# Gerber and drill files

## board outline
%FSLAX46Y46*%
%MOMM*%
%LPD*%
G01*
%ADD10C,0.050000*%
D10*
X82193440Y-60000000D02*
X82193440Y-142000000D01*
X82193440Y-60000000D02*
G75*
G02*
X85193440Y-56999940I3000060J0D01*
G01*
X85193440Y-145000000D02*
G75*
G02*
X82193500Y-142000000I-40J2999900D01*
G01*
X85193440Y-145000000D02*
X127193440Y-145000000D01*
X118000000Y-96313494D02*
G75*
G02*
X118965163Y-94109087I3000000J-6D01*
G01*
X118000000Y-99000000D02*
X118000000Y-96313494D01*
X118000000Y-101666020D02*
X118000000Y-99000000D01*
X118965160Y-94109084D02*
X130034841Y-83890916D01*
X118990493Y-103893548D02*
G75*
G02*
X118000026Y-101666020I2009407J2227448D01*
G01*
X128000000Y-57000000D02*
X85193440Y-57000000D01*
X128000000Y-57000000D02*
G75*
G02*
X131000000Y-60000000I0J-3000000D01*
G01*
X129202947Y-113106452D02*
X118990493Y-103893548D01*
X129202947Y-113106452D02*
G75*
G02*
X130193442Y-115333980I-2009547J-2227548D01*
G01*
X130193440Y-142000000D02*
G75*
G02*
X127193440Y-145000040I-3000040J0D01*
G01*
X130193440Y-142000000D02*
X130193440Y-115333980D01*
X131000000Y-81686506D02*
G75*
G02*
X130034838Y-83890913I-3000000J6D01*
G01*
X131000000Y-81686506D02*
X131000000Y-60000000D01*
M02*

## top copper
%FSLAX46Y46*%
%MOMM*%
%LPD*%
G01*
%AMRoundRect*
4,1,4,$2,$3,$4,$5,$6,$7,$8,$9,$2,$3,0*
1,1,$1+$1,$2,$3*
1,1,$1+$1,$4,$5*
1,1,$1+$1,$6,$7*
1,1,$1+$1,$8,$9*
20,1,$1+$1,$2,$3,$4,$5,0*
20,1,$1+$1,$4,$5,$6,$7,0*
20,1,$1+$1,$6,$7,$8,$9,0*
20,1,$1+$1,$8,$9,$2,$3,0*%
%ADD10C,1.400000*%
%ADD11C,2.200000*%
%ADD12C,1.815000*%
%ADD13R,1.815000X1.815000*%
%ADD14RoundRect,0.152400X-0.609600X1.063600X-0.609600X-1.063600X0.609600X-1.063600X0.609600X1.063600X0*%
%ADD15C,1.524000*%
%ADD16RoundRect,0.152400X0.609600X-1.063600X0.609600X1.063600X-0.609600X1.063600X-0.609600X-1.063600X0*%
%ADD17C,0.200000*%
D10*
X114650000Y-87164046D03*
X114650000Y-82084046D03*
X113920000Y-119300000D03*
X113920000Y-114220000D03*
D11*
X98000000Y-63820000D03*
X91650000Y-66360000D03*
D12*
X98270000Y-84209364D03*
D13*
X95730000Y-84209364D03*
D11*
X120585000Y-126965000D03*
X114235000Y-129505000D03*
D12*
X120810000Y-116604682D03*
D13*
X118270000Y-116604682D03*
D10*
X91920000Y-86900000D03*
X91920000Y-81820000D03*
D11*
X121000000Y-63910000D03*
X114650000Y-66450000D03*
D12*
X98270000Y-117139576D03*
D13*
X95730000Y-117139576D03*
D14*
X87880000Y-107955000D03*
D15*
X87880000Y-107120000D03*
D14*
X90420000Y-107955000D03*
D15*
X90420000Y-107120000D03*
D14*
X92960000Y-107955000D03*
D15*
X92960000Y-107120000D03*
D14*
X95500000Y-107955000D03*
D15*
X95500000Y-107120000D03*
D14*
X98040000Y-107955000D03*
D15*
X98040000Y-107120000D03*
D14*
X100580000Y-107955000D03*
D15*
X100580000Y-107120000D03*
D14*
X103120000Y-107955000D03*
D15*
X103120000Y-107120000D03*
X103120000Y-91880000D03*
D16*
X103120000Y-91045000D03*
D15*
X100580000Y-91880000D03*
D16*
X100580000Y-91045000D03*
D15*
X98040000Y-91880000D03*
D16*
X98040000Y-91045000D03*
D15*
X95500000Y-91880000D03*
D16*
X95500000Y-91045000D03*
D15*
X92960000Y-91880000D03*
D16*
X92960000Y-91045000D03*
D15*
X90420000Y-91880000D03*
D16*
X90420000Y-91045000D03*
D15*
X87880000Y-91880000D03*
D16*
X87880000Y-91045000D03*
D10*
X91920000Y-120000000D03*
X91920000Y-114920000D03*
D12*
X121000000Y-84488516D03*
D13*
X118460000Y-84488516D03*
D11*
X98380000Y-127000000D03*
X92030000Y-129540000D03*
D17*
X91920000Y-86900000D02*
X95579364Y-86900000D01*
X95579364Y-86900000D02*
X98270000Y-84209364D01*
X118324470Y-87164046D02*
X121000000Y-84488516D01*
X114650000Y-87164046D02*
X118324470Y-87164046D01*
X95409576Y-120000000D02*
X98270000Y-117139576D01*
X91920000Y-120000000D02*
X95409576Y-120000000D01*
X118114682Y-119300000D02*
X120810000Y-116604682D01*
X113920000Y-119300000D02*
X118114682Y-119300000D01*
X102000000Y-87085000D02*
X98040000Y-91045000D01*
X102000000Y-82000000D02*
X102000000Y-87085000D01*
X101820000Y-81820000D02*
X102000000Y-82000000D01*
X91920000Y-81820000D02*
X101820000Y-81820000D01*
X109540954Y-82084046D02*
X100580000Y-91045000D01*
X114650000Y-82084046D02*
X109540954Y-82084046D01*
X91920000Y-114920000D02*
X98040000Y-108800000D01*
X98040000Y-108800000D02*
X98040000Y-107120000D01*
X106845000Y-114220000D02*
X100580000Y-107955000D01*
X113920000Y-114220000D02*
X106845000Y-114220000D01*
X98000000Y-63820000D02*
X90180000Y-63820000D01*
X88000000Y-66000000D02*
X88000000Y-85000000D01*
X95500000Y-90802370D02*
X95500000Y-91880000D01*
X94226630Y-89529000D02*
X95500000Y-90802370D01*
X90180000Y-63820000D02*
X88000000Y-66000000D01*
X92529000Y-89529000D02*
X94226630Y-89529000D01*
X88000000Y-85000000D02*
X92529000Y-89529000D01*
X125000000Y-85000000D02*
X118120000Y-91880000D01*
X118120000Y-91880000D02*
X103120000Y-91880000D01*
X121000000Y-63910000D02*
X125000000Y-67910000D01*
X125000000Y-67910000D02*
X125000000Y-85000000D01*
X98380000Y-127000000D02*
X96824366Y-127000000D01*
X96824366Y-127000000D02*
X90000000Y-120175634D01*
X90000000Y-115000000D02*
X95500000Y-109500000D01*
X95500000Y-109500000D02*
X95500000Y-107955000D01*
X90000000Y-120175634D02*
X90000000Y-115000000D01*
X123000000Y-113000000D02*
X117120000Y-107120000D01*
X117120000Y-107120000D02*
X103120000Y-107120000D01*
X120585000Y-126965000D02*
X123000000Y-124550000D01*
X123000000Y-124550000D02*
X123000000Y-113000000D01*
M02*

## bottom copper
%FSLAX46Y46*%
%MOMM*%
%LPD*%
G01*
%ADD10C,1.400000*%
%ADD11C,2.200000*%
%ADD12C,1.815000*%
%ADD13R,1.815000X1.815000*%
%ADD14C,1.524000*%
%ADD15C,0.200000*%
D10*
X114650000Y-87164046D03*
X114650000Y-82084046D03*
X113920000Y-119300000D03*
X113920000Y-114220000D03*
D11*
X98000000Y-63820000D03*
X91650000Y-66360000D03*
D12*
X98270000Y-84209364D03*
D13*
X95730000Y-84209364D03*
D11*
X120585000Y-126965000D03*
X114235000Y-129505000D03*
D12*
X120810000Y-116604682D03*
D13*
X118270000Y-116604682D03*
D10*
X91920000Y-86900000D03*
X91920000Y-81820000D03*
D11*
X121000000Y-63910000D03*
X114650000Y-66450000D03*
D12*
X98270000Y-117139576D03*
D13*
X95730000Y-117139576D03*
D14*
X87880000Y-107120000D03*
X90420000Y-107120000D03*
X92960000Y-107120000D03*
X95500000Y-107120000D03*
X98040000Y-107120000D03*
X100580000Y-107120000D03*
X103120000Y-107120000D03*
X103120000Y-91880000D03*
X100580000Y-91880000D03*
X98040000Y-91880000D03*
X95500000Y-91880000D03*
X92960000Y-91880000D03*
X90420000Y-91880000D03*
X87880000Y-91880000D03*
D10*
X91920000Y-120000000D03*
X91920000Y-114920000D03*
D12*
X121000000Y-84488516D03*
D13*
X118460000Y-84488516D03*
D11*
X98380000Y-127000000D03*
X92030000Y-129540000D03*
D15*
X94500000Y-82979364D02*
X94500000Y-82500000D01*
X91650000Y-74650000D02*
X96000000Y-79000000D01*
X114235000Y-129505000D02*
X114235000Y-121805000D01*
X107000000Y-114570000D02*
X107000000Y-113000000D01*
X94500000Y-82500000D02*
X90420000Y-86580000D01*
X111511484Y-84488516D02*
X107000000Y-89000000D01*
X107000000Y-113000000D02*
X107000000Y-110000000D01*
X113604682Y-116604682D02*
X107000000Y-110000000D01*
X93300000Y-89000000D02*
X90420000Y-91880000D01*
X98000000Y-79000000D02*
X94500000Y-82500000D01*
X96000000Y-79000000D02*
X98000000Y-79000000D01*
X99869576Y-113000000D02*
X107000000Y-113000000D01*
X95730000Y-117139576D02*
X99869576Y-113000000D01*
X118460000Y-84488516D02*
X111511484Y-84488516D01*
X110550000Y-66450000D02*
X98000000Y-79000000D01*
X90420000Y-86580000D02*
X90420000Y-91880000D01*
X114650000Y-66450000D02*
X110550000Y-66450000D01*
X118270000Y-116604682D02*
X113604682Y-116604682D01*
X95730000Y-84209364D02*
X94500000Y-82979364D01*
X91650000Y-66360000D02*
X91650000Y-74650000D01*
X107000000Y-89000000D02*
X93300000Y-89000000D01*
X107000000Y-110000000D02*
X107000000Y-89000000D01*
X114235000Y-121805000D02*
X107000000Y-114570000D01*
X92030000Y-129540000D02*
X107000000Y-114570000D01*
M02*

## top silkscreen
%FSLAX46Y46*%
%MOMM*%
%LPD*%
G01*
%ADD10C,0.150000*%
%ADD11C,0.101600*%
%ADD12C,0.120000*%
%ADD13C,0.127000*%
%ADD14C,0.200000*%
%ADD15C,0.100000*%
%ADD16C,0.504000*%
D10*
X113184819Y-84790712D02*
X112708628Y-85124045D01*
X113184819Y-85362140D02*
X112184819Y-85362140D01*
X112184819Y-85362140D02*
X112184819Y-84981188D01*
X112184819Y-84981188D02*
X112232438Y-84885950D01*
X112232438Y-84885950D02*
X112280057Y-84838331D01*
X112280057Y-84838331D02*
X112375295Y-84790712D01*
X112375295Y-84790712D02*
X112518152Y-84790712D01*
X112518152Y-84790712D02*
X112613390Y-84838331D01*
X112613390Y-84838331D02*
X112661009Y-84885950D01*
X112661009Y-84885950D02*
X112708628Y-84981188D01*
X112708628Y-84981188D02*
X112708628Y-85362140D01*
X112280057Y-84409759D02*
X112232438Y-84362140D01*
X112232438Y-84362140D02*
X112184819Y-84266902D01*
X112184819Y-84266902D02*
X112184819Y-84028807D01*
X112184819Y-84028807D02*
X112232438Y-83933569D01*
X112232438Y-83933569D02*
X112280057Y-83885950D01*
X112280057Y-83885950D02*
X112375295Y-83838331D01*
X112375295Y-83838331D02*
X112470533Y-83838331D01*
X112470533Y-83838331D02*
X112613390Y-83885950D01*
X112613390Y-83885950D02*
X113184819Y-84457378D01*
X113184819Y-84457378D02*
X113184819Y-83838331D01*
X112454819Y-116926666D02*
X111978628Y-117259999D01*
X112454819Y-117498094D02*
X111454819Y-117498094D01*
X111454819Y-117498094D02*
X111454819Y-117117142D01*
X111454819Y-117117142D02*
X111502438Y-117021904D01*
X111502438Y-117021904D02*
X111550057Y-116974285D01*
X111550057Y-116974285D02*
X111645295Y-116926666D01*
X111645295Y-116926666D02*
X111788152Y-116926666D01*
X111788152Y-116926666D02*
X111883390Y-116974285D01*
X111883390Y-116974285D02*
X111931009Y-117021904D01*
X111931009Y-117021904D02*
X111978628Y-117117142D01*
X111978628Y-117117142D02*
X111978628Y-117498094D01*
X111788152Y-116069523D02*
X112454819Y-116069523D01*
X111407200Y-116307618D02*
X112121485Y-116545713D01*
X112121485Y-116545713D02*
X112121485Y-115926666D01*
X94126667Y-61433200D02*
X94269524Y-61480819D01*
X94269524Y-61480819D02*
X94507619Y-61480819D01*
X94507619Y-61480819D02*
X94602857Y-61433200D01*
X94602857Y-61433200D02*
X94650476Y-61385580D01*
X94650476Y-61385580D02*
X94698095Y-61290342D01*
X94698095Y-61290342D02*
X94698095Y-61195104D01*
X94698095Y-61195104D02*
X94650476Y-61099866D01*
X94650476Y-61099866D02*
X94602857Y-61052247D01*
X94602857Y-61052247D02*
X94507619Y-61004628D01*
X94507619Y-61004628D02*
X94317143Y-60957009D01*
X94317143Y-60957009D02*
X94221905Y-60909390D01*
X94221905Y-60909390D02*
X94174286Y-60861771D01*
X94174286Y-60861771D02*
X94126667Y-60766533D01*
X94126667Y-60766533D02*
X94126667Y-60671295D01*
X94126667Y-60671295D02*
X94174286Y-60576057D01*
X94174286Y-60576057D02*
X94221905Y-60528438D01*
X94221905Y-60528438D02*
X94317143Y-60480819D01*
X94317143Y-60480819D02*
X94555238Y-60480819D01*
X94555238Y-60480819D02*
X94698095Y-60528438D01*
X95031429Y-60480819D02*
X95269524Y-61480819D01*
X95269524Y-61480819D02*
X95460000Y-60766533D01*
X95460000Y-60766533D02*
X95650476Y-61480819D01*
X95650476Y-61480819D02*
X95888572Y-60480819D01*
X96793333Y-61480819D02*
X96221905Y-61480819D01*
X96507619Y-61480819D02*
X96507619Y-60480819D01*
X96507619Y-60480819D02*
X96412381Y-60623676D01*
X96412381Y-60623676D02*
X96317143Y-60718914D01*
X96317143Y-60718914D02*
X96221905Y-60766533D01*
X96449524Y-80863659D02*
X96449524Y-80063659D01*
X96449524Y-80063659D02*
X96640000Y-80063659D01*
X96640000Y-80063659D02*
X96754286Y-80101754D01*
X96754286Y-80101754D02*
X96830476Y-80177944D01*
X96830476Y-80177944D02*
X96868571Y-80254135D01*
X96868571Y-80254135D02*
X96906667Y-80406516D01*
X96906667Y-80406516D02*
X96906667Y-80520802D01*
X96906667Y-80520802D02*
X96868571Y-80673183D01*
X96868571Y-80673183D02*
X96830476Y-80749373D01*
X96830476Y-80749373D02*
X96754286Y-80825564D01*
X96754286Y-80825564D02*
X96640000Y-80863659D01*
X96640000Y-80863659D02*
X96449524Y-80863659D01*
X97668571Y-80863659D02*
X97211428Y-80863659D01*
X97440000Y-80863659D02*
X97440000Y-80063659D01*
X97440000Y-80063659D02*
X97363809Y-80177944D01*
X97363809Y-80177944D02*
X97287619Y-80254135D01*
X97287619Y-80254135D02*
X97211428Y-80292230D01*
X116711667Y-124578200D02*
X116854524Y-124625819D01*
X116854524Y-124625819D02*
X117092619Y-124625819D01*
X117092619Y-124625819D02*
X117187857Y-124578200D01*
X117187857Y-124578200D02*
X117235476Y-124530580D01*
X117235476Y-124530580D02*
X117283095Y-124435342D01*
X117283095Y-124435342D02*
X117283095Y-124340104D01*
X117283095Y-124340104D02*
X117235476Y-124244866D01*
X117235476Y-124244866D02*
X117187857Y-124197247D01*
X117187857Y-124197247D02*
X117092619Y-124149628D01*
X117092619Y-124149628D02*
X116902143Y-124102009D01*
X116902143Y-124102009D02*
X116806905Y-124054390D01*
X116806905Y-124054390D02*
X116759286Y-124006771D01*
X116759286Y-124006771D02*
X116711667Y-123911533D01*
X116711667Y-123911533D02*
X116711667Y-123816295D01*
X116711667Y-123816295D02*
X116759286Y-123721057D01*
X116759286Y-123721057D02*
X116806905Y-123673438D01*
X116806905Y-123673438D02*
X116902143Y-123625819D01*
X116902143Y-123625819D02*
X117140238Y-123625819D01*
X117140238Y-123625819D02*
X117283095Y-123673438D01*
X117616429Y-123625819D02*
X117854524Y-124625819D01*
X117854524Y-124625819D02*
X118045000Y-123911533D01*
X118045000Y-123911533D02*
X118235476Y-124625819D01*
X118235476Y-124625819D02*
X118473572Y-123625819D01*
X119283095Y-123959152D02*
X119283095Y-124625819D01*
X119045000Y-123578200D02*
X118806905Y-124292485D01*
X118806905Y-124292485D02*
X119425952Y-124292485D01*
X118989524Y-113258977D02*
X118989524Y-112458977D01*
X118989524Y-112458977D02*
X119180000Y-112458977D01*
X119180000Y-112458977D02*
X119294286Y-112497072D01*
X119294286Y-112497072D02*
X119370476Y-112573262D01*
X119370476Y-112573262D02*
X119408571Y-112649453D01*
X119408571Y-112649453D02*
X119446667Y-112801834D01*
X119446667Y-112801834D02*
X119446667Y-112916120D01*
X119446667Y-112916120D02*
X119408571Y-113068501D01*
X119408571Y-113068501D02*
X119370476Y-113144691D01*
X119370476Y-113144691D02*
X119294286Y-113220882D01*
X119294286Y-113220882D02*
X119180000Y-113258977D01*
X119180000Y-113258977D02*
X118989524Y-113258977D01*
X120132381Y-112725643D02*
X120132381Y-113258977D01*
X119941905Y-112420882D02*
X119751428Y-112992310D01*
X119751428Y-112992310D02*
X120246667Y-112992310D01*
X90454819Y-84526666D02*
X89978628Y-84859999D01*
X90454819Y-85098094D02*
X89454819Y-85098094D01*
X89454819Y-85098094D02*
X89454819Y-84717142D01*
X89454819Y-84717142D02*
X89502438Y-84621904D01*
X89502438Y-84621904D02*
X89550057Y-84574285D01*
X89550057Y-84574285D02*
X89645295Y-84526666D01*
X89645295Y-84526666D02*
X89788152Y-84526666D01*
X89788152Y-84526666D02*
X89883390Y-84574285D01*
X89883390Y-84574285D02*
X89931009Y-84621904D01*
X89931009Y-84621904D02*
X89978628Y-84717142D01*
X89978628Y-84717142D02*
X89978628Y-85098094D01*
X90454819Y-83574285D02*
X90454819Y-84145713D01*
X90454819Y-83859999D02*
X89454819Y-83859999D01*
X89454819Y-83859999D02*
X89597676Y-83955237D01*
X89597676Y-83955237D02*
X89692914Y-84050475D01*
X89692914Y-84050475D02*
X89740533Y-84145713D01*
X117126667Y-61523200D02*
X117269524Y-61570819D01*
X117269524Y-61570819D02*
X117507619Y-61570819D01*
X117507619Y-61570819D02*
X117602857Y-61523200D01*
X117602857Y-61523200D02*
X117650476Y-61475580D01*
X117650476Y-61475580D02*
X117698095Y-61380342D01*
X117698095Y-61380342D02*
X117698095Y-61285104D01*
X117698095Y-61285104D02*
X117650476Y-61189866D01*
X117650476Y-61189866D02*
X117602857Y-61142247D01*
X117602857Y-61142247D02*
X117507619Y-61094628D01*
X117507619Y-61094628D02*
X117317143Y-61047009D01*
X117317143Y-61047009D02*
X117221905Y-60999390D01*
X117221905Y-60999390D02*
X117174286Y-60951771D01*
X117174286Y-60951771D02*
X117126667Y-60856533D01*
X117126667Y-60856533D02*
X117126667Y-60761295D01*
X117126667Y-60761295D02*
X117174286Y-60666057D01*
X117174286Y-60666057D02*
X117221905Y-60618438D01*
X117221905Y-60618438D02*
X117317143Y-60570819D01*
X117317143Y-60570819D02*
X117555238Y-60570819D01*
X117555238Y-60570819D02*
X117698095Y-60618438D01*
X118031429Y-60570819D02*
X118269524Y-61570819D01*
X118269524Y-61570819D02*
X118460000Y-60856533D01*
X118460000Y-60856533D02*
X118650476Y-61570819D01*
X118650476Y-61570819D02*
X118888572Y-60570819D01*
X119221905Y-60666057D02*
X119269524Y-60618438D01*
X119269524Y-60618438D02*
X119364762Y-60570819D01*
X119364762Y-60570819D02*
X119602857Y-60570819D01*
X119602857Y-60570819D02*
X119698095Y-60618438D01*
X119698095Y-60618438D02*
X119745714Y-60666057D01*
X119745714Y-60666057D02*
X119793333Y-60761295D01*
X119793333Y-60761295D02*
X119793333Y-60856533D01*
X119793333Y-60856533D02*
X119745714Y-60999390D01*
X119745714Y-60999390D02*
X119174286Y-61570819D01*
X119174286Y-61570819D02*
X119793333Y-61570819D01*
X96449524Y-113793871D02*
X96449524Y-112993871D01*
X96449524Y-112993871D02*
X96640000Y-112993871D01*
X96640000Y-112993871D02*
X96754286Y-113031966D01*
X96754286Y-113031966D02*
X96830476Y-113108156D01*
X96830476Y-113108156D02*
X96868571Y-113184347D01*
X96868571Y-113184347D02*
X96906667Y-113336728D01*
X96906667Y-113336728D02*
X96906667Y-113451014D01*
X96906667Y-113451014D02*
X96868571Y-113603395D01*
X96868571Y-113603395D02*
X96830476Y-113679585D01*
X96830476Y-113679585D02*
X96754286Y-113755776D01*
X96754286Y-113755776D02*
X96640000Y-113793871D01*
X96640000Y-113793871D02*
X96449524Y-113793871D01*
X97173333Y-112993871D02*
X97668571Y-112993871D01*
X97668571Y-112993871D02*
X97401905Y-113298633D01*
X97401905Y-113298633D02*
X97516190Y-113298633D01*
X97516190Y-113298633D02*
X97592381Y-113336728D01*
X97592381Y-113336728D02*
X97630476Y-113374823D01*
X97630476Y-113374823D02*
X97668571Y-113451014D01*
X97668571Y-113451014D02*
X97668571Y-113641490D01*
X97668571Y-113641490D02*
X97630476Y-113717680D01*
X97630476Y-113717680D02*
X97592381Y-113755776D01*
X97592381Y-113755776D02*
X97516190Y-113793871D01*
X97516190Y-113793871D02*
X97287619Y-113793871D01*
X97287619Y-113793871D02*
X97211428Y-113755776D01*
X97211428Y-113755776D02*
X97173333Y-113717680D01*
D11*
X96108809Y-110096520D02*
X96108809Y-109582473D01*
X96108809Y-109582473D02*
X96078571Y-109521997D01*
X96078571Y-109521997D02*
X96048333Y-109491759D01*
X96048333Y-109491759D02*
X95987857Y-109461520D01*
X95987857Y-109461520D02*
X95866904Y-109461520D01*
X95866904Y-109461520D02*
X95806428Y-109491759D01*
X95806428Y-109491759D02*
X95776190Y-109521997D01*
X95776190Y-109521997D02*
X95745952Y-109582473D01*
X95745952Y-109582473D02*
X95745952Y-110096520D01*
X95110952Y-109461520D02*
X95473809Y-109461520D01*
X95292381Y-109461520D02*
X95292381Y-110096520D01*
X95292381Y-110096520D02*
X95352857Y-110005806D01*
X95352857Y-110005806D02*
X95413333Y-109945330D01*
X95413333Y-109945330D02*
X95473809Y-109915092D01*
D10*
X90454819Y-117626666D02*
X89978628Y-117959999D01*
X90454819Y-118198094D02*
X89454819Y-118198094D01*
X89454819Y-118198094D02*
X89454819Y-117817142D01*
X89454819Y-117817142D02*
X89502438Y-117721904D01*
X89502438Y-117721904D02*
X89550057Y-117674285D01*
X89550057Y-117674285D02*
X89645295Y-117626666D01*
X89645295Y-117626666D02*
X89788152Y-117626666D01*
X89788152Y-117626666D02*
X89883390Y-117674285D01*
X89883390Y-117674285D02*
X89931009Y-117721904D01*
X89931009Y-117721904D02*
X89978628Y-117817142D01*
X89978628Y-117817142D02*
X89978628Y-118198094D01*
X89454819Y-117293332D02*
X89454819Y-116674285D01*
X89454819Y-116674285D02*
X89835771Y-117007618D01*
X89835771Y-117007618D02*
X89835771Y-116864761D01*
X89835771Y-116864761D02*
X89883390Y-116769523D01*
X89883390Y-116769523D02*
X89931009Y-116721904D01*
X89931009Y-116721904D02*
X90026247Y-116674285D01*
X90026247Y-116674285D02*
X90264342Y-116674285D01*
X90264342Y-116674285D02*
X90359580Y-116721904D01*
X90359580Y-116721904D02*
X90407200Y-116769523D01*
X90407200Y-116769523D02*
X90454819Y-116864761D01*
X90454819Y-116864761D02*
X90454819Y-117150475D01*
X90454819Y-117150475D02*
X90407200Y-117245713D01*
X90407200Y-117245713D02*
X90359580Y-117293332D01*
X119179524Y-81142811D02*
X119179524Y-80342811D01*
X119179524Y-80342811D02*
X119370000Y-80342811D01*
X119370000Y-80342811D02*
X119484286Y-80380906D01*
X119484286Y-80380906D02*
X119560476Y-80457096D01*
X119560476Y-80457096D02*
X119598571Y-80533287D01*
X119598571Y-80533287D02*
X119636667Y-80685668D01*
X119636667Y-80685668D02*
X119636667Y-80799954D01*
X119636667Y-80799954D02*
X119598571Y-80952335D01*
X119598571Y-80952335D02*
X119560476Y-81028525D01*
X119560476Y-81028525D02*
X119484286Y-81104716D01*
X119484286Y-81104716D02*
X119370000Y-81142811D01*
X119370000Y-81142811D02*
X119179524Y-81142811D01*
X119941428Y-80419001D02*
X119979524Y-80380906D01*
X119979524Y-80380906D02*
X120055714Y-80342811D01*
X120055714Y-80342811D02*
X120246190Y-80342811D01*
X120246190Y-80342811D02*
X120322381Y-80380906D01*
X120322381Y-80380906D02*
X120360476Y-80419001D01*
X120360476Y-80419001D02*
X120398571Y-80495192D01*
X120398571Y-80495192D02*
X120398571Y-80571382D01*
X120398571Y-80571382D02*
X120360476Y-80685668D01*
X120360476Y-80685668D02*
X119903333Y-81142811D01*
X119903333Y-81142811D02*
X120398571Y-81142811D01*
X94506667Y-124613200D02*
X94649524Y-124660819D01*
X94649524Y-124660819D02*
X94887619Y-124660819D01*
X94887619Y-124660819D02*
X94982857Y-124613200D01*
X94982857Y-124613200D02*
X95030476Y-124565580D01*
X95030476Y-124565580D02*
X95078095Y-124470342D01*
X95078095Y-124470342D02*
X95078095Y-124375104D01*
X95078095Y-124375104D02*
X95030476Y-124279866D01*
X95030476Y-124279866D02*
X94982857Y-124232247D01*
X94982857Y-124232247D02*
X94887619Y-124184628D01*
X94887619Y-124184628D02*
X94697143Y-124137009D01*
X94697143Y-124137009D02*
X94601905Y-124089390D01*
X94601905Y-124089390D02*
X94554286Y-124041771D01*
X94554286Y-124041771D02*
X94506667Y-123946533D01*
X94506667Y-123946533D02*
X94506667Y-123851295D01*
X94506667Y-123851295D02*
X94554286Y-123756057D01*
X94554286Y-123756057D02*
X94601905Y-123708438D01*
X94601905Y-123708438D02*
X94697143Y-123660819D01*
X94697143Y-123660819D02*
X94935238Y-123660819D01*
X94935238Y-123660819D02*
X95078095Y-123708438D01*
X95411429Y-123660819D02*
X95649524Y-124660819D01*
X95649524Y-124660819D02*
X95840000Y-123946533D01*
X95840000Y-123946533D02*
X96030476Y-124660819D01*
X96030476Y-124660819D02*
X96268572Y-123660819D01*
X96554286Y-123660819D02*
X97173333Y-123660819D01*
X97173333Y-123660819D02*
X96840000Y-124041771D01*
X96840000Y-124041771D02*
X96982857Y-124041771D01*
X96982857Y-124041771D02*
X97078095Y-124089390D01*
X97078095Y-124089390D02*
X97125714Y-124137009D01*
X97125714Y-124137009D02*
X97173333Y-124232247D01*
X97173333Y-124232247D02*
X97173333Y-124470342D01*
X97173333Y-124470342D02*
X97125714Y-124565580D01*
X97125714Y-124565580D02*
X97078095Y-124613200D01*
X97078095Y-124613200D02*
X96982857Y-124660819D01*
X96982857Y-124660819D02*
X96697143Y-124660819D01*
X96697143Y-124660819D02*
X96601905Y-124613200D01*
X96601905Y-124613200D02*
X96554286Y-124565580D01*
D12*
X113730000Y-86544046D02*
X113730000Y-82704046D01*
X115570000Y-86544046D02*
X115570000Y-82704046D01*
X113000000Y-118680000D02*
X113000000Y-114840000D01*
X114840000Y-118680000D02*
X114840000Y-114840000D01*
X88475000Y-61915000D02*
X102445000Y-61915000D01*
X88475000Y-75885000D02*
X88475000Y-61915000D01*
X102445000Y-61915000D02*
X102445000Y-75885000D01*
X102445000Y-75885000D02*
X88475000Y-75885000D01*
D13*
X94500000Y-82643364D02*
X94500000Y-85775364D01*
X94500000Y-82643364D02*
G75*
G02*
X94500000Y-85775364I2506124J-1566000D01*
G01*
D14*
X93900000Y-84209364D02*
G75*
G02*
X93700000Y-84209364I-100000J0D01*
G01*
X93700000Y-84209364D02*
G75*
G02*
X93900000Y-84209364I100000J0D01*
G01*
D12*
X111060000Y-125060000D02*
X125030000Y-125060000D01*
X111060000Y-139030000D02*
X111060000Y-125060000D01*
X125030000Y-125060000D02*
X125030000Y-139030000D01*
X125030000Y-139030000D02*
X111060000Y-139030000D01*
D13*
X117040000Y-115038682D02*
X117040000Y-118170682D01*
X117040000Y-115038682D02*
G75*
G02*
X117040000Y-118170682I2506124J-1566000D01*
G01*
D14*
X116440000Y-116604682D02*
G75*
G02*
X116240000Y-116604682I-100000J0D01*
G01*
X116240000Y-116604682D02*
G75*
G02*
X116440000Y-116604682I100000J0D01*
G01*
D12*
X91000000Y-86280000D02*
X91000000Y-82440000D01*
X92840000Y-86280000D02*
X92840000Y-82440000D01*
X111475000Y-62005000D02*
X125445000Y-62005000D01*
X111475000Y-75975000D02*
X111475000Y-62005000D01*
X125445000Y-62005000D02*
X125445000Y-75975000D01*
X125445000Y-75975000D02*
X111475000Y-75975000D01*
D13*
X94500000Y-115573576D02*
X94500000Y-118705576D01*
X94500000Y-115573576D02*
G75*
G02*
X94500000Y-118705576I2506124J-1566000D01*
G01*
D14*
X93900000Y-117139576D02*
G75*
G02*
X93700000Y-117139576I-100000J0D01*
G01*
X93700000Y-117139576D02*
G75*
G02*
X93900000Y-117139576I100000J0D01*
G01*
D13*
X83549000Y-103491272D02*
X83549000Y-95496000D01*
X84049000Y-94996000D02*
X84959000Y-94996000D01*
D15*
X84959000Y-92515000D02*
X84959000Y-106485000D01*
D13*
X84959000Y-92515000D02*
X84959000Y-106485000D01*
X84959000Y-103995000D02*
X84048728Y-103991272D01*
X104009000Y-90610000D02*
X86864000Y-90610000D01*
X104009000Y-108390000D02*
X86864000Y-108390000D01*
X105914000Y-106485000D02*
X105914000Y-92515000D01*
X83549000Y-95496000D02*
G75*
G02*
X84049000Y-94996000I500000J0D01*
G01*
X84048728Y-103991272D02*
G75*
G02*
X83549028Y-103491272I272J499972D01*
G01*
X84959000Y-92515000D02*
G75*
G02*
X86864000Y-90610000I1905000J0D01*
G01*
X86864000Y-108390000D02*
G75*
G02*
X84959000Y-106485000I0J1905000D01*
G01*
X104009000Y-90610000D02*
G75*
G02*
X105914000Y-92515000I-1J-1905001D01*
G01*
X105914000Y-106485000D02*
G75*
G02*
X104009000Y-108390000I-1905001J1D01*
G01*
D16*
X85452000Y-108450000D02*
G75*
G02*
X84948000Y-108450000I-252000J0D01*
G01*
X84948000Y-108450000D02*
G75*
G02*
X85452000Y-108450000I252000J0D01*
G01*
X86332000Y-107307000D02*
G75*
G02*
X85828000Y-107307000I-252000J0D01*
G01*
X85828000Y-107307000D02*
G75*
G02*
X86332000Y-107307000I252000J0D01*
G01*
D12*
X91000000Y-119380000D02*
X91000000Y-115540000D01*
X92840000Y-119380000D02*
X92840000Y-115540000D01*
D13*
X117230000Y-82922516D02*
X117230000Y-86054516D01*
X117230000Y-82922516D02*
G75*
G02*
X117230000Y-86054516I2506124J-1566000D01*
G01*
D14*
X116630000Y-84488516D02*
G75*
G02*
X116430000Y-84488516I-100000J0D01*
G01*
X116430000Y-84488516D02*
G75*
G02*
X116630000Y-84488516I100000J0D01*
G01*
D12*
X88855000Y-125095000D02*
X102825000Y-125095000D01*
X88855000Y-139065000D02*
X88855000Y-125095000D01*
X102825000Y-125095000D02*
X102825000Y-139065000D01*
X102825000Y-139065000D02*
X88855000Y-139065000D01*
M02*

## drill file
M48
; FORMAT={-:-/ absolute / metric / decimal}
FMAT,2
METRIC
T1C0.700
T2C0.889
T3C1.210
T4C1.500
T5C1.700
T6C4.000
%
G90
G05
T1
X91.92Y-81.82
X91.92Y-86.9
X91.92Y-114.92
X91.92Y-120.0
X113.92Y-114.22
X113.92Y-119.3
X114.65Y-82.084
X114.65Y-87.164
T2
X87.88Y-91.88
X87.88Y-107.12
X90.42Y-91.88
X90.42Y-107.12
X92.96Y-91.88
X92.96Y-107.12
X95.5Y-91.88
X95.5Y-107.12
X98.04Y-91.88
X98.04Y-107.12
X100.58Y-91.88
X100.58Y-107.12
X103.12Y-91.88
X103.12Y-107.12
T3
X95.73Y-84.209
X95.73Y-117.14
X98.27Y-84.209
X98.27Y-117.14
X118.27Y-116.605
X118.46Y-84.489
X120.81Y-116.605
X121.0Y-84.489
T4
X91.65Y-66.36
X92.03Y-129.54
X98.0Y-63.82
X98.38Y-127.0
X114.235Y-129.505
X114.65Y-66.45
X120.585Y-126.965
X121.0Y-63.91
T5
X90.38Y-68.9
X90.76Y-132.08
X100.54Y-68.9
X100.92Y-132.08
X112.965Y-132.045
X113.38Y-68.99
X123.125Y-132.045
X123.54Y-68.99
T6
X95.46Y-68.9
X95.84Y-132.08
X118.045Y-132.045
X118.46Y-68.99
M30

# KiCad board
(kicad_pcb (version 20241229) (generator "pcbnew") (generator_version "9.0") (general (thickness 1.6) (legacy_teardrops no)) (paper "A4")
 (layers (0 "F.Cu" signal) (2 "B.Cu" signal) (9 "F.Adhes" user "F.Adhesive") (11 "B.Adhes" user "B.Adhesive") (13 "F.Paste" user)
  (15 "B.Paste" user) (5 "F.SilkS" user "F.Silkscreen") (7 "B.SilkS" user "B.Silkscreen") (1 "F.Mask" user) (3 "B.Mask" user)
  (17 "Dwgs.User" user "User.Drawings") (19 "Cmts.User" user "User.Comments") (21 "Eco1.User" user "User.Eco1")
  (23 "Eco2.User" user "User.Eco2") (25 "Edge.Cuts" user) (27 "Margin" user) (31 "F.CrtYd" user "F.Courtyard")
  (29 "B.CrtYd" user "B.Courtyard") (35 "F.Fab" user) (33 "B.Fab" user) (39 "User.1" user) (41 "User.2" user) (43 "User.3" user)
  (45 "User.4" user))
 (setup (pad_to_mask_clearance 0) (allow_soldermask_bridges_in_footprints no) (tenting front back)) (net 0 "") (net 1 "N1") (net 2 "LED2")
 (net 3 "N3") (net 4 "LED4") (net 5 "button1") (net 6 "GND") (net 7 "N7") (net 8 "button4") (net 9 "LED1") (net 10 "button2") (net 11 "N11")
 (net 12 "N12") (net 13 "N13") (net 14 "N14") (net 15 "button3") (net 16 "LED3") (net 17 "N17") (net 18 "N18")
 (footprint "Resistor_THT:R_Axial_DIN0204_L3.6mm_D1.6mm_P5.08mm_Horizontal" (layer "F.Cu") (at 114.65 87.164046 90)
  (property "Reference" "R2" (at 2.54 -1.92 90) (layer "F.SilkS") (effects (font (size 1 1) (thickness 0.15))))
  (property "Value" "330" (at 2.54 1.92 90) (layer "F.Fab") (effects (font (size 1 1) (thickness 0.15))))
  (fp_line (start 0.62 -0.92) (end 4.46 -0.92) (stroke (width 0.12) (type solid)) (layer "F.SilkS"))
  (fp_line (start 0.62 0.92) (end 4.46 0.92) (stroke (width 0.12) (type solid)) (layer "F.SilkS"))
  (pad "1" thru_hole circle (at 0 0 90) (size 1.4 1.4) (drill 0.7) (layers "*.Cu" "*.Mask") (remove_unused_layers no) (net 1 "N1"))
  (pad "2" thru_hole circle (at 5.08 0 90) (size 1.4 1.4) (drill 0.7) (layers "*.Cu" "*.Mask") (remove_unused_layers no) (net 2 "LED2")))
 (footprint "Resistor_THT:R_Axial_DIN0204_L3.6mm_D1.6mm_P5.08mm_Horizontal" (layer "F.Cu") (at 113.92 119.3 90)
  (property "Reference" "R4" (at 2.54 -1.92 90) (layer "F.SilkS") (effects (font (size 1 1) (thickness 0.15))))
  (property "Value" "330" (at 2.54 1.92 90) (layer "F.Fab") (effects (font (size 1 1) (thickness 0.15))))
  (fp_line (start 0.62 -0.92) (end 4.46 -0.92) (stroke (width 0.12) (type solid)) (layer "F.SilkS"))
  (fp_line (start 0.62 0.92) (end 4.46 0.92) (stroke (width 0.12) (type solid)) (layer "F.SilkS"))
  (pad "1" thru_hole circle (at 0 0 90) (size 1.4 1.4) (drill 0.7) (layers "*.Cu" "*.Mask") (remove_unused_layers no) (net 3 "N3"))
  (pad "2" thru_hole circle (at 5.08 0 90) (size 1.4 1.4) (drill 0.7) (layers "*.Cu" "*.Mask") (remove_unused_layers no) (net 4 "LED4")))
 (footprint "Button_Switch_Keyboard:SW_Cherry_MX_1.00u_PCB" (layer "F.Cu") (at 98 63.82)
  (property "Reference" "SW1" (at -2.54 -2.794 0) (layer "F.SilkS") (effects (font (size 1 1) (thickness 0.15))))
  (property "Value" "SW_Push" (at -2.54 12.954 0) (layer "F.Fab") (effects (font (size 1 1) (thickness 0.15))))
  (fp_line (start -9.525 -1.905) (end 4.445 -1.905) (stroke (width 0.12) (type solid)) (layer "F.SilkS"))
  (fp_line (start -9.525 12.065) (end -9.525 -1.905) (stroke (width 0.12) (type solid)) (layer "F.SilkS"))
  (fp_line (start 4.445 -1.905) (end 4.445 12.065) (stroke (width 0.12) (type solid)) (layer "F.SilkS"))
  (fp_line (start 4.445 12.065) (end -9.525 12.065) (stroke (width 0.12) (type solid)) (layer "F.SilkS"))
  (pad "" np_thru_hole circle (at -7.62 5.08) (size 1.7 1.7) (drill 1.7) (layers "*.Cu" "*.Mask"))
  (pad "" np_thru_hole circle (at -2.54 5.08) (size 4 4) (drill 4) (layers "*.Cu" "*.Mask"))
  (pad "" np_thru_hole circle (at 2.54 5.08) (size 1.7 1.7) (drill 1.7) (layers "*.Cu" "*.Mask"))
  (pad "1" thru_hole circle (at 0 0) (size 2.2 2.2) (drill 1.5) (layers "*.Cu" "*.Mask") (remove_unused_layers no) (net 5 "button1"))
  (pad "2" thru_hole circle (at -6.35 2.54) (size 2.2 2.2) (drill 1.5) (layers "*.Cu" "*.Mask") (remove_unused_layers no) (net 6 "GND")))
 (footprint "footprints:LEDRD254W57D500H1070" (layer "F.Cu") (at 97 84.209364)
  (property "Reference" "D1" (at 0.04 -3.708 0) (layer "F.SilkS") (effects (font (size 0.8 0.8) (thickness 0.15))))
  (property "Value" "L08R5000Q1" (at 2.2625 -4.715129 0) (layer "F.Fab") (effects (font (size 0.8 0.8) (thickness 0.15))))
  (fp_line (start -2.5 -1.566) (end -2.5 1.566) (stroke (width 0.127) (type solid)) (layer "F.SilkS"))
  (fp_arc (start -2.5 -1.566) (mid 2.961291 0) (end -2.5 1.566) (stroke (width 0.127) (type solid)) (layer "F.SilkS"))
  (fp_circle (center -3.2 0) (end -3.1 0) (stroke (width 0.2) (type solid)) (fill no) (layer "F.SilkS"))
  (pad "A" thru_hole circle (at 1.27 0) (size 1.815 1.815) (drill 1.21) (layers "*.Cu" "*.Mask") (remove_unused_layers no) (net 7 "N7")
   (solder_mask_margin 0.102))
  (pad "C" thru_hole rect (at -1.27 0) (size 1.815 1.815) (drill 1.21) (layers "*.Cu" "*.Mask") (remove_unused_layers no) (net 6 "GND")
   (solder_mask_margin 0.102)))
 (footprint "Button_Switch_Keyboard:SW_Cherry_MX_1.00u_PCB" (layer "F.Cu") (at 120.585 126.965)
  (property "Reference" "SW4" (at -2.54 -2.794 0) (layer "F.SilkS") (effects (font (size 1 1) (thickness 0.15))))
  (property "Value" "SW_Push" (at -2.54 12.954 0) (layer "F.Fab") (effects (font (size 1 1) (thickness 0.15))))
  (fp_line (start -9.525 -1.905) (end 4.445 -1.905) (stroke (width 0.12) (type solid)) (layer "F.SilkS"))
  (fp_line (start -9.525 12.065) (end -9.525 -1.905) (stroke (width 0.12) (type solid)) (layer "F.SilkS"))
  (fp_line (start 4.445 -1.905) (end 4.445 12.065) (stroke (width 0.12) (type solid)) (layer "F.SilkS"))
  (fp_line (start 4.445 12.065) (end -9.525 12.065) (stroke (width 0.12) (type solid)) (layer "F.SilkS"))
  (pad "" np_thru_hole circle (at -7.62 5.08) (size 1.7 1.7) (drill 1.7) (layers "*.Cu" "*.Mask"))
  (pad "" np_thru_hole circle (at -2.54 5.08) (size 4 4) (drill 4) (layers "*.Cu" "*.Mask"))
  (pad "" np_thru_hole circle (at 2.54 5.08) (size 1.7 1.7) (drill 1.7) (layers "*.Cu" "*.Mask"))
  (pad "1" thru_hole circle (at 0 0) (size 2.2 2.2) (drill 1.5) (layers "*.Cu" "*.Mask") (remove_unused_layers no) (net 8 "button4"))
  (pad "2" thru_hole circle (at -6.35 2.54) (size 2.2 2.2) (drill 1.5) (layers "*.Cu" "*.Mask") (remove_unused_layers no) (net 6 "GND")))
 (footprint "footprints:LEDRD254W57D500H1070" (layer "F.Cu") (at 119.54 116.604682)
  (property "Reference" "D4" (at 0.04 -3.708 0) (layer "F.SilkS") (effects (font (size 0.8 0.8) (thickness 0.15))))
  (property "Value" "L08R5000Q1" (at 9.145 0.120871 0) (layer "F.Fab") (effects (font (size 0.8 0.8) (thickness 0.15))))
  (fp_line (start -2.5 -1.566) (end -2.5 1.566) (stroke (width 0.127) (type solid)) (layer "F.SilkS"))
  (fp_arc (start -2.5 -1.566) (mid 2.961291 0) (end -2.5 1.566) (stroke (width 0.127) (type solid)) (layer "F.SilkS"))
  (fp_circle (center -3.2 0) (end -3.1 0) (stroke (width 0.2) (type solid)) (fill no) (layer "F.SilkS"))
  (pad "A" thru_hole circle (at 1.27 0) (size 1.815 1.815) (drill 1.21) (layers "*.Cu" "*.Mask") (remove_unused_layers no) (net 3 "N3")
   (solder_mask_margin 0.102))
  (pad "C" thru_hole rect (at -1.27 0) (size 1.815 1.815) (drill 1.21) (layers "*.Cu" "*.Mask") (remove_unused_layers no) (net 6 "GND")
   (solder_mask_margin 0.102)))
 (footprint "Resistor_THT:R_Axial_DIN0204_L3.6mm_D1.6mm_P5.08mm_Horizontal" (layer "F.Cu") (at 91.92 86.9 90)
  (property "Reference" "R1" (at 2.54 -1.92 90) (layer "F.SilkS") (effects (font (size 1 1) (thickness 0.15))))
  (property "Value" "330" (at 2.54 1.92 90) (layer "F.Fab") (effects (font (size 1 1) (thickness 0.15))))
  (fp_line (start 0.62 -0.92) (end 4.46 -0.92) (stroke (width 0.12) (type solid)) (layer "F.SilkS"))
  (fp_line (start 0.62 0.92) (end 4.46 0.92) (stroke (width 0.12) (type solid)) (layer "F.SilkS"))
  (pad "1" thru_hole circle (at 0 0 90) (size 1.4 1.4) (drill 0.7) (layers "*.Cu" "*.Mask") (remove_unused_layers no) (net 7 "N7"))
  (pad "2" thru_hole circle (at 5.08 0 90) (size 1.4 1.4) (drill 0.7) (layers "*.Cu" "*.Mask") (remove_unused_layers no) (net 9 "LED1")))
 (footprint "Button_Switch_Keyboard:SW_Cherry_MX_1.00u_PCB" (layer "F.Cu") (at 121 63.91)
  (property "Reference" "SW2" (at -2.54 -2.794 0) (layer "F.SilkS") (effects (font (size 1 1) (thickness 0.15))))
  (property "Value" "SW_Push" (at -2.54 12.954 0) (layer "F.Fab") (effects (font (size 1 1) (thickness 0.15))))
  (fp_line (start -9.525 -1.905) (end 4.445 -1.905) (stroke (width 0.12) (type solid)) (layer "F.SilkS"))
  (fp_line (start -9.525 12.065) (end -9.525 -1.905) (stroke (width 0.12) (type solid)) (layer "F.SilkS"))
  (fp_line (start 4.445 -1.905) (end 4.445 12.065) (stroke (width 0.12) (type solid)) (layer "F.SilkS"))
  (fp_line (start 4.445 12.065) (end -9.525 12.065) (stroke (width 0.12) (type solid)) (layer "F.SilkS"))
  (pad "" np_thru_hole circle (at -7.62 5.08) (size 1.7 1.7) (drill 1.7) (layers "*.Cu" "*.Mask"))
  (pad "" np_thru_hole circle (at -2.54 5.08) (size 4 4) (drill 4) (layers "*.Cu" "*.Mask"))
  (pad "" np_thru_hole circle (at 2.54 5.08) (size 1.7 1.7) (drill 1.7) (layers "*.Cu" "*.Mask"))
  (pad "1" thru_hole circle (at 0 0) (size 2.2 2.2) (drill 1.5) (layers "*.Cu" "*.Mask") (remove_unused_layers no) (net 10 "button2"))
  (pad "2" thru_hole circle (at -6.35 2.54) (size 2.2 2.2) (drill 1.5) (layers "*.Cu" "*.Mask") (remove_unused_layers no) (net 6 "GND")))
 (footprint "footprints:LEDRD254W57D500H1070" (layer "F.Cu") (at 97 117.139576)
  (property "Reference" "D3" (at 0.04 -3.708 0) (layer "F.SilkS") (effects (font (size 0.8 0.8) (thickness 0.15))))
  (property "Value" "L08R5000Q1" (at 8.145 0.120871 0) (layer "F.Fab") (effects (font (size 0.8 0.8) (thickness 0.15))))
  (fp_line (start -2.5 -1.566) (end -2.5 1.566) (stroke (width 0.127) (type solid)) (layer "F.SilkS"))
  (fp_arc (start -2.5 -1.566) (mid 2.961291 0) (end -2.5 1.566) (stroke (width 0.127) (type solid)) (layer "F.SilkS"))
  (fp_circle (center -3.2 0) (end -3.1 0) (stroke (width 0.2) (type solid)) (fill no) (layer "F.SilkS"))
  (pad "A" thru_hole circle (at 1.27 0) (size 1.815 1.815) (drill 1.21) (layers "*.Cu" "*.Mask") (remove_unused_layers no) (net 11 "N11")
   (solder_mask_margin 0.102))
  (pad "C" thru_hole rect (at -1.27 0) (size 1.815 1.815) (drill 1.21) (layers "*.Cu" "*.Mask") (remove_unused_layers no) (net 6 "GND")
   (solder_mask_margin 0.102)))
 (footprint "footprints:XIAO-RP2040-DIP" (layer "F.Cu") (at 95.5 99.5 180)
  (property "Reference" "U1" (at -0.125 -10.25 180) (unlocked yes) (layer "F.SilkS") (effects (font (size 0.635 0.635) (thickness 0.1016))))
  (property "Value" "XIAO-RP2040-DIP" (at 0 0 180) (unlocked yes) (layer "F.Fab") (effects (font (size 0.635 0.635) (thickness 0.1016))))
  (fp_line (start 11.951 -3.991272) (end 11.951 4.004) (stroke (width 0.127) (type solid)) (layer "F.SilkS"))
  (fp_line (start 11.451 4.504) (end 10.541 4.504) (stroke (width 0.127) (type solid)) (layer "F.SilkS"))
  (fp_line (start 10.541 6.985) (end 10.541 -6.985) (stroke (width 0.1) (type solid)) (layer "F.SilkS"))
  (fp_line (start 10.541 6.985) (end 10.541 -6.985) (stroke (width 0.127) (type solid)) (layer "F.SilkS"))
  (fp_line (start 10.541 -4.495) (end 11.451272 -4.491272) (stroke (width 0.127) (type solid)) (layer "F.SilkS"))
  (fp_line (start -8.509 8.89) (end 8.636 8.89) (stroke (width 0.127) (type solid)) (layer "F.SilkS"))
  (fp_line (start -8.509 -8.89) (end 8.636 -8.89) (stroke (width 0.127) (type solid)) (layer "F.SilkS"))
  (fp_line (start -10.414 -6.985) (end -10.414 6.985) (stroke (width 0.127) (type solid)) (layer "F.SilkS"))
  (fp_arc (start 11.951 4.004) (mid 11.804553 4.357553) (end 11.451 4.504) (stroke (width 0.127) (type default)) (layer "F.SilkS"))
  (fp_arc (start 11.451272 -4.491272) (mid 11.804644 -4.344724) (end 11.951 -3.991272) (stroke (width 0.127) (type default))
   (layer "F.SilkS"))
  (fp_arc (start 10.541 6.985) (mid 9.983038 8.332038) (end 8.636 8.89) (stroke (width 0.127) (type solid)) (layer "F.SilkS"))
  (fp_arc (start 8.636 -8.89) (mid 9.983038 -8.332038) (end 10.541 -6.985) (stroke (width 0.127) (type solid)) (layer "F.SilkS"))
  (fp_arc (start -8.509 8.89) (mid -9.856038 8.332038) (end -10.414 6.985) (stroke (width 0.127) (type solid)) (layer "F.SilkS"))
  (fp_arc (start -10.414 -6.985) (mid -9.856038 -8.332038) (end -8.509 -8.89) (stroke (width 0.127) (type solid)) (layer "F.SilkS"))
  (fp_circle (center 10.3 -8.95) (end 10.554 -8.95) (stroke (width 0.5) (type solid)) (fill yes) (layer "F.SilkS"))
  (fp_circle (center 9.42 -7.807) (end 9.674 -7.807) (stroke (width 0.5) (type solid)) (fill yes) (layer "F.SilkS"))
  (pad "1" smd roundrect (at 7.62 -8.455 270) (size 2.432 1.524) (layers "F.Cu" "F.Mask") (roundrect_rratio 0.1) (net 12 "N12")
   (thermal_bridge_angle 45))
  (pad "1" thru_hole circle (at 7.62 -7.62 270) (size 1.524 1.524) (drill 0.889) (layers "*.Cu" "*.Mask") (remove_unused_layers no)
   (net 12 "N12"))
  (pad "2" smd roundrect (at 5.08 -8.455 270) (size 2.432 1.524) (layers "F.Cu" "F.Mask") (roundrect_rratio 0.1) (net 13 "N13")
   (thermal_bridge_angle 45))
  (pad "2" thru_hole circle (at 5.08 -7.62 270) (size 1.524 1.524) (drill 0.889) (layers "*.Cu" "*.Mask") (remove_unused_layers no)
   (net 13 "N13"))
  (pad "3" smd roundrect (at 2.54 -8.455 270) (size 2.432 1.524) (layers "F.Cu" "F.Mask") (roundrect_rratio 0.1) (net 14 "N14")
   (thermal_bridge_angle 45))
  (pad "3" thru_hole circle (at 2.54 -7.62 270) (size 1.524 1.524) (drill 0.889) (layers "*.Cu" "*.Mask") (remove_unused_layers no)
   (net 14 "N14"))
  (pad "4" smd roundrect (at 0 -8.455 270) (size 2.432 1.524) (layers "F.Cu" "F.Mask") (roundrect_rratio 0.1) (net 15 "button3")
   (thermal_bridge_angle 45))
  (pad "4" thru_hole circle (at 0 -7.62 270) (size 1.524 1.524) (drill 0.889) (layers "*.Cu" "*.Mask") (remove_unused_layers no)
   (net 15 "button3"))
  (pad "5" smd roundrect (at -2.54 -8.455 270) (size 2.432 1.524) (layers "F.Cu" "F.Mask") (roundrect_rratio 0.1) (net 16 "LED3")
   (thermal_bridge_angle 45))
  (pad "5" thru_hole circle (at -2.54 -7.62 270) (size 1.524 1.524) (drill 0.889) (layers "*.Cu" "*.Mask") (remove_unused_layers no)
   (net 16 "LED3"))
  (pad "6" smd roundrect (at -5.08 -8.455 270) (size 2.432 1.524) (layers "F.Cu" "F.Mask") (roundrect_rratio 0.1) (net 4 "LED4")
   (thermal_bridge_angle 45))
  (pad "6" thru_hole circle (at -5.08 -7.62 270) (size 1.524 1.524) (drill 0.889) (layers "*.Cu" "*.Mask") (remove_unused_layers no)
   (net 4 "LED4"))
  (pad "7" smd roundrect (at -7.62 -8.455 270) (size 2.432 1.524) (layers "F.Cu" "F.Mask") (roundrect_rratio 0.1) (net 8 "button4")
   (thermal_bridge_angle 45))
  (pad "7" thru_hole circle (at -7.62 -7.62 270) (size 1.524 1.524) (drill 0.889) (layers "*.Cu" "*.Mask") (remove_unused_layers no)
   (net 8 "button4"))
  (pad "8" thru_hole circle (at -7.62 7.62 90) (size 1.524 1.524) (drill 0.889) (layers "*.Cu" "*.Mask") (remove_unused_layers no)
   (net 10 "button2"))
  (pad "8" smd roundrect (at -7.62 8.455 90) (size 2.432 1.524) (layers "F.Cu" "F.Mask") (roundrect_rratio 0.1) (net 10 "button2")
   (thermal_bridge_angle 45))
  (pad "9" thru_hole circle (at -5.08 7.62 90) (size 1.524 1.524) (drill 0.889) (layers "*.Cu" "*.Mask") (remove_unused_layers no)
   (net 2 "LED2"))
  (pad "9" smd roundrect (at -5.08 8.455 90) (size 2.432 1.524) (layers "F.Cu" "F.Mask") (roundrect_rratio 0.1) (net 2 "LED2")
   (thermal_bridge_angle 45))
  (pad "10" thru_hole circle (at -2.54 7.62 90) (size 1.524 1.524) (drill 0.889) (layers "*.Cu" "*.Mask") (remove_unused_layers no)
   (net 9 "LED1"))
  (pad "10" smd roundrect (at -2.54 8.455 90) (size 2.432 1.524) (layers "F.Cu" "F.Mask") (roundrect_rratio 0.1) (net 9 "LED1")
   (thermal_bridge_angle 45))
  (pad "11" thru_hole circle (at 0 7.62 90) (size 1.524 1.524) (drill 0.889) (layers "*.Cu" "*.Mask") (remove_unused_layers no)
   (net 5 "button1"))
  (pad "11" smd roundrect (at 0 8.455 90) (size 2.432 1.524) (layers "F.Cu" "F.Mask") (roundrect_rratio 0.1) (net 5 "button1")
   (thermal_bridge_angle 45))
  (pad "12" thru_hole circle (at 2.54 7.62 90) (size 1.524 1.524) (drill 0.889) (layers "*.Cu" "*.Mask") (remove_unused_layers no)
   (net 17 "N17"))
  (pad "12" smd roundrect (at 2.54 8.455 90) (size 2.432 1.524) (layers "F.Cu" "F.Mask") (roundrect_rratio 0.1) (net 17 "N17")
   (thermal_bridge_angle 45))
  (pad "13" thru_hole circle (at 5.08 7.62 90) (size 1.524 1.524) (drill 0.889) (layers "*.Cu" "*.Mask") (remove_unused_layers no)
   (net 6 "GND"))
  (pad "13" smd roundrect (at 5.08 8.455 90) (size 2.432 1.524) (layers "F.Cu" "F.Mask") (roundrect_rratio 0.1) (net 6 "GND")
   (thermal_bridge_angle 45))
  (pad "14" thru_hole circle (at 7.62 7.62 90) (size 1.524 1.524) (drill 0.889) (layers "*.Cu" "*.Mask") (remove_unused_layers no)
   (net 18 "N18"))
  (pad "14" smd roundrect (at 7.62 8.455 90) (size 2.432 1.524) (layers "F.Cu" "F.Mask") (roundrect_rratio 0.1) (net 18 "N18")
   (thermal_bridge_angle 45)))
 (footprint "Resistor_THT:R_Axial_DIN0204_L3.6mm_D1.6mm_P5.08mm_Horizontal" (layer "F.Cu") (at 91.92 120 90)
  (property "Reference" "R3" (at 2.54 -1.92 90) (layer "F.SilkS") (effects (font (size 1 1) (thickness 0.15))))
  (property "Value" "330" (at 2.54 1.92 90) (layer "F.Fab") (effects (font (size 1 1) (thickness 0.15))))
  (fp_line (start 0.62 -0.92) (end 4.46 -0.92) (stroke (width 0.12) (type solid)) (layer "F.SilkS"))
  (fp_line (start 0.62 0.92) (end 4.46 0.92) (stroke (width 0.12) (type solid)) (layer "F.SilkS"))
  (pad "1" thru_hole circle (at 0 0 90) (size 1.4 1.4) (drill 0.7) (layers "*.Cu" "*.Mask") (remove_unused_layers no) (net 11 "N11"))
  (pad "2" thru_hole circle (at 5.08 0 90) (size 1.4 1.4) (drill 0.7) (layers "*.Cu" "*.Mask") (remove_unused_layers no) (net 16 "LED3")))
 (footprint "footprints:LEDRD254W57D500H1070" (layer "F.Cu") (at 119.73 84.488516)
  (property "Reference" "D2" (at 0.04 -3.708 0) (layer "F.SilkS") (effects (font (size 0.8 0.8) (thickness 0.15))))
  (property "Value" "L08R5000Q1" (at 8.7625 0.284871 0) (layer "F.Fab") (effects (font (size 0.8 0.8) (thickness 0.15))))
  (fp_line (start -2.5 -1.566) (end -2.5 1.566) (stroke (width 0.127) (type solid)) (layer "F.SilkS"))
  (fp_arc (start -2.5 -1.566) (mid 2.961291 0) (end -2.5 1.566) (stroke (width 0.127) (type solid)) (layer "F.SilkS"))
  (fp_circle (center -3.2 0) (end -3.1 0) (stroke (width 0.2) (type solid)) (fill no) (layer "F.SilkS"))
  (pad "A" thru_hole circle (at 1.27 0) (size 1.815 1.815) (drill 1.21) (layers "*.Cu" "*.Mask") (remove_unused_layers no) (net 1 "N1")
   (solder_mask_margin 0.102))
  (pad "C" thru_hole rect (at -1.27 0) (size 1.815 1.815) (drill 1.21) (layers "*.Cu" "*.Mask") (remove_unused_layers no) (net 6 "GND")
   (solder_mask_margin 0.102)))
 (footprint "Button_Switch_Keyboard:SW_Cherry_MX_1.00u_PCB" (layer "F.Cu") (at 98.38 127)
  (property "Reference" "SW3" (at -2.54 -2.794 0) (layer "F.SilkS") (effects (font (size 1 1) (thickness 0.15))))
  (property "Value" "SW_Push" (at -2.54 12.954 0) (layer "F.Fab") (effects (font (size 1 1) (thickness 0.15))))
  (fp_line (start -9.525 -1.905) (end 4.445 -1.905) (stroke (width 0.12) (type solid)) (layer "F.SilkS"))
  (fp_line (start -9.525 12.065) (end -9.525 -1.905) (stroke (width 0.12) (type solid)) (layer "F.SilkS"))
  (fp_line (start 4.445 -1.905) (end 4.445 12.065) (stroke (width 0.12) (type solid)) (layer "F.SilkS"))
  (fp_line (start 4.445 12.065) (end -9.525 12.065) (stroke (width 0.12) (type solid)) (layer "F.SilkS"))
  (pad "" np_thru_hole circle (at -7.62 5.08) (size 1.7 1.7) (drill 1.7) (layers "*.Cu" "*.Mask"))
  (pad "" np_thru_hole circle (at -2.54 5.08) (size 4 4) (drill 4) (layers "*.Cu" "*.Mask"))
  (pad "" np_thru_hole circle (at 2.54 5.08) (size 1.7 1.7) (drill 1.7) (layers "*.Cu" "*.Mask"))
  (pad "1" thru_hole circle (at 0 0) (size 2.2 2.2) (drill 1.5) (layers "*.Cu" "*.Mask") (remove_unused_layers no) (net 15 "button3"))
  (pad "2" thru_hole circle (at -6.35 2.54) (size 2.2 2.2) (drill 1.5) (layers "*.Cu" "*.Mask") (remove_unused_layers no) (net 6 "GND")))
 (gr_line (start 82.19344 60) (end 82.19344 142) (stroke (width 0.05) (type default)) (layer "Edge.Cuts"))
 (gr_arc (start 82.19344 60) (mid 83.072122 57.878694) (end 85.19344 57) (stroke (width 0.05) (type default)) (layer "Edge.Cuts"))
 (gr_arc (start 85.19344 145) (mid 83.072094 144.121334) (end 82.19344 142) (stroke (width 0.05) (type default)) (layer "Edge.Cuts"))
 (gr_line (start 85.19344 145) (end 127.19344 145) (stroke (width 0.05) (type default)) (layer "Edge.Cuts"))
 (gr_arc (start 118 96.313494) (mid 118.251864 95.110275) (end 118.96516 94.109084) (stroke (width 0.05) (type default)) (layer "Edge.Cuts"))
 (gr_line (start 118 99) (end 118 96.313494) (stroke (width 0.05) (type default)) (layer "Edge.Cuts"))
 (gr_line (start 118 101.66602) (end 118 99) (stroke (width 0.05) (type default)) (layer "Edge.Cuts"))
 (gr_line (start 118.96516 94.109084) (end 130.034841 83.890916) (stroke (width 0.05) (type default)) (layer "Edge.Cuts"))
 (gr_arc (start 118.990493 103.893548) (mid 118.258778 102.88493) (end 118 101.66602) (stroke (width 0.05) (type default))
  (layer "Edge.Cuts"))
 (gr_line (start 128 57) (end 85.19344 57) (stroke (width 0.05) (type default)) (layer "Edge.Cuts"))
 (gr_arc (start 128 57) (mid 130.12132 57.87868) (end 131 60) (stroke (width 0.05) (type default)) (layer "Edge.Cuts"))
 (gr_line (start 129.202947 113.106452) (end 118.990493 103.893548) (stroke (width 0.05) (type default)) (layer "Edge.Cuts"))
 (gr_arc (start 129.202947 113.106452) (mid 129.934652 114.115072) (end 130.19344 115.33398) (stroke (width 0.05) (type default))
  (layer "Edge.Cuts"))
 (gr_arc (start 130.19344 142) (mid 129.314757 144.121299) (end 127.19344 145) (stroke (width 0.05) (type default)) (layer "Edge.Cuts"))
 (gr_line (start 130.19344 142) (end 130.19344 115.33398) (stroke (width 0.05) (type default)) (layer "Edge.Cuts"))
 (gr_arc (start 131 81.686506) (mid 130.748136 82.889725) (end 130.034841 83.890916) (stroke (width 0.05) (type default))
  (layer "Edge.Cuts"))
 (gr_line (start 131 81.686506) (end 131 60) (stroke (width 0.05) (type default)) (layer "Edge.Cuts"))
 (segment (start 91.92 86.9) (end 95.579364 86.9) (width 0.2) (layer "F.Cu") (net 7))
 (segment (start 95.579364 86.9) (end 98.27 84.209364) (width 0.2) (layer "F.Cu") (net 7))
 (segment (start 94.5 82.979364) (end 94.5 82.5) (width 0.2) (layer "B.Cu") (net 6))
 (segment (start 91.65 74.65) (end 96 79) (width 0.2) (layer "B.Cu") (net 6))
 (segment (start 114.235 129.505) (end 114.235 121.805) (width 0.2) (layer "B.Cu") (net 6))
 (segment (start 107 114.57) (end 107 113) (width 0.2) (layer "B.Cu") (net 6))
 (segment (start 94.5 82.5) (end 90.42 86.58) (width 0.2) (layer "B.Cu") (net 6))
 (segment (start 111.511484 84.488516) (end 107 89) (width 0.2) (layer "B.Cu") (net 6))
 (segment (start 107 113) (end 107 110) (width 0.2) (layer "B.Cu") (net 6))
 (segment (start 113.604682 116.604682) (end 107 110) (width 0.2) (layer "B.Cu") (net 6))
 (segment (start 93.3 89) (end 90.42 91.88) (width 0.2) (layer "B.Cu") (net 6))
 (segment (start 98 79) (end 94.5 82.5) (width 0.2) (layer "B.Cu") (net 6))
 (segment (start 96 79) (end 98 79) (width 0.2) (layer "B.Cu") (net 6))
 (segment (start 99.869576 113) (end 107 113) (width 0.2) (layer "B.Cu") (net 6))
 (segment (start 95.73 117.139576) (end 99.869576 113) (width 0.2) (layer "B.Cu") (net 6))
 (segment (start 118.46 84.488516) (end 111.511484 84.488516) (width 0.2) (layer "B.Cu") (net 6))
 (segment (start 110.55 66.45) (end 98 79) (width 0.2) (layer "B.Cu") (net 6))
 (segment (start 90.42 86.58) (end 90.42 91.88) (width 0.2) (layer "B.Cu") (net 6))
 (segment (start 114.65 66.45) (end 110.55 66.45) (width 0.2) (layer "B.Cu") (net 6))
 (segment (start 118.27 116.604682) (end 113.604682 116.604682) (width 0.2) (layer "B.Cu") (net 6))
 (segment (start 95.73 84.209364) (end 94.5 82.979364) (width 0.2) (layer "B.Cu") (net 6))
 (segment (start 91.65 66.36) (end 91.65 74.65) (width 0.2) (layer "B.Cu") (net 6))
 (segment (start 107 89) (end 93.3 89) (width 0.2) (layer "B.Cu") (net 6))
 (segment (start 107 110) (end 107 89) (width 0.2) (layer "B.Cu") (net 6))
 (segment (start 114.235 121.805) (end 107 114.57) (width 0.2) (layer "B.Cu") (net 6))
 (segment (start 92.03 129.54) (end 107 114.57) (width 0.2) (layer "B.Cu") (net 6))
 (segment (start 118.32447 87.164046) (end 121 84.488516) (width 0.2) (layer "F.Cu") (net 1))
 (segment (start 114.65 87.164046) (end 118.32447 87.164046) (width 0.2) (layer "F.Cu") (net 1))
 (segment (start 95.409576 120) (end 98.27 117.139576) (width 0.2) (layer "F.Cu") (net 11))
 (segment (start 91.92 120) (end 95.409576 120) (width 0.2) (layer "F.Cu") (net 11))
 (segment (start 118.114682 119.3) (end 120.81 116.604682) (width 0.2) (layer "F.Cu") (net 3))
 (segment (start 113.92 119.3) (end 118.114682 119.3) (width 0.2) (layer "F.Cu") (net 3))
 (segment (start 102 87.085) (end 98.04 91.045) (width 0.2) (layer "F.Cu") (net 9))
 (segment (start 102 82) (end 102 87.085) (width 0.2) (layer "F.Cu") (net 9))
 (segment (start 101.82 81.82) (end 102 82) (width 0.2) (layer "F.Cu") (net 9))
 (segment (start 91.92 81.82) (end 101.82 81.82) (width 0.2) (layer "F.Cu") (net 9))
 (segment (start 109.540954 82.084046) (end 100.58 91.045) (width 0.2) (layer "F.Cu") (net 2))
 (segment (start 114.65 82.084046) (end 109.540954 82.084046) (width 0.2) (layer "F.Cu") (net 2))
 (segment (start 91.92 114.92) (end 98.04 108.8) (width 0.2) (layer "F.Cu") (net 16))
 (segment (start 98.04 108.8) (end 98.04 107.12) (width 0.2) (layer "F.Cu") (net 16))
 (segment (start 106.845 114.22) (end 100.58 107.955) (width 0.2) (layer "F.Cu") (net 4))
 (segment (start 113.92 114.22) (end 106.845 114.22) (width 0.2) (layer "F.Cu") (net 4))
 (segment (start 98 63.82) (end 90.18 63.82) (width 0.2) (layer "F.Cu") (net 5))
 (segment (start 88 66) (end 88 85) (width 0.2) (layer "F.Cu") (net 5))
 (segment (start 95.5 90.80237) (end 95.5 91.88) (width 0.2) (layer "F.Cu") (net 5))
 (segment (start 94.22663 89.529) (end 95.5 90.80237) (width 0.2) (layer "F.Cu") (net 5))
 (segment (start 90.18 63.82) (end 88 66) (width 0.2) (layer "F.Cu") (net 5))
 (segment (start 92.529 89.529) (end 94.22663 89.529) (width 0.2) (layer "F.Cu") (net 5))
 (segment (start 88 85) (end 92.529 89.529) (width 0.2) (layer "F.Cu") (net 5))
 (segment (start 125 85) (end 118.12 91.88) (width 0.2) (layer "F.Cu") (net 10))
 (segment (start 118.12 91.88) (end 103.12 91.88) (width 0.2) (layer "F.Cu") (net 10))
 (segment (start 121 63.91) (end 125 67.91) (width 0.2) (layer "F.Cu") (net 10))
 (segment (start 125 67.91) (end 125 85) (width 0.2) (layer "F.Cu") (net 10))
 (segment (start 98.38 127) (end 96.824366 127) (width 0.2) (layer "F.Cu") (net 15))
 (segment (start 96.824366 127) (end 90 120.175634) (width 0.2) (layer "F.Cu") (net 15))
 (segment (start 90 115) (end 95.5 109.5) (width 0.2) (layer "F.Cu") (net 15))
 (segment (start 95.5 109.5) (end 95.5 107.955) (width 0.2) (layer "F.Cu") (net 15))
 (segment (start 90 120.175634) (end 90 115) (width 0.2) (layer "F.Cu") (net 15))
 (segment (start 123 113) (end 117.12 107.12) (width 0.2) (layer "F.Cu") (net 8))
 (segment (start 117.12 107.12) (end 103.12 107.12) (width 0.2) (layer "F.Cu") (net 8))
 (segment (start 120.585 126.965) (end 123 124.55) (width 0.2) (layer "F.Cu") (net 8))
 (segment (start 123 124.55) (end 123 113) (width 0.2) (layer "F.Cu") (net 8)))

